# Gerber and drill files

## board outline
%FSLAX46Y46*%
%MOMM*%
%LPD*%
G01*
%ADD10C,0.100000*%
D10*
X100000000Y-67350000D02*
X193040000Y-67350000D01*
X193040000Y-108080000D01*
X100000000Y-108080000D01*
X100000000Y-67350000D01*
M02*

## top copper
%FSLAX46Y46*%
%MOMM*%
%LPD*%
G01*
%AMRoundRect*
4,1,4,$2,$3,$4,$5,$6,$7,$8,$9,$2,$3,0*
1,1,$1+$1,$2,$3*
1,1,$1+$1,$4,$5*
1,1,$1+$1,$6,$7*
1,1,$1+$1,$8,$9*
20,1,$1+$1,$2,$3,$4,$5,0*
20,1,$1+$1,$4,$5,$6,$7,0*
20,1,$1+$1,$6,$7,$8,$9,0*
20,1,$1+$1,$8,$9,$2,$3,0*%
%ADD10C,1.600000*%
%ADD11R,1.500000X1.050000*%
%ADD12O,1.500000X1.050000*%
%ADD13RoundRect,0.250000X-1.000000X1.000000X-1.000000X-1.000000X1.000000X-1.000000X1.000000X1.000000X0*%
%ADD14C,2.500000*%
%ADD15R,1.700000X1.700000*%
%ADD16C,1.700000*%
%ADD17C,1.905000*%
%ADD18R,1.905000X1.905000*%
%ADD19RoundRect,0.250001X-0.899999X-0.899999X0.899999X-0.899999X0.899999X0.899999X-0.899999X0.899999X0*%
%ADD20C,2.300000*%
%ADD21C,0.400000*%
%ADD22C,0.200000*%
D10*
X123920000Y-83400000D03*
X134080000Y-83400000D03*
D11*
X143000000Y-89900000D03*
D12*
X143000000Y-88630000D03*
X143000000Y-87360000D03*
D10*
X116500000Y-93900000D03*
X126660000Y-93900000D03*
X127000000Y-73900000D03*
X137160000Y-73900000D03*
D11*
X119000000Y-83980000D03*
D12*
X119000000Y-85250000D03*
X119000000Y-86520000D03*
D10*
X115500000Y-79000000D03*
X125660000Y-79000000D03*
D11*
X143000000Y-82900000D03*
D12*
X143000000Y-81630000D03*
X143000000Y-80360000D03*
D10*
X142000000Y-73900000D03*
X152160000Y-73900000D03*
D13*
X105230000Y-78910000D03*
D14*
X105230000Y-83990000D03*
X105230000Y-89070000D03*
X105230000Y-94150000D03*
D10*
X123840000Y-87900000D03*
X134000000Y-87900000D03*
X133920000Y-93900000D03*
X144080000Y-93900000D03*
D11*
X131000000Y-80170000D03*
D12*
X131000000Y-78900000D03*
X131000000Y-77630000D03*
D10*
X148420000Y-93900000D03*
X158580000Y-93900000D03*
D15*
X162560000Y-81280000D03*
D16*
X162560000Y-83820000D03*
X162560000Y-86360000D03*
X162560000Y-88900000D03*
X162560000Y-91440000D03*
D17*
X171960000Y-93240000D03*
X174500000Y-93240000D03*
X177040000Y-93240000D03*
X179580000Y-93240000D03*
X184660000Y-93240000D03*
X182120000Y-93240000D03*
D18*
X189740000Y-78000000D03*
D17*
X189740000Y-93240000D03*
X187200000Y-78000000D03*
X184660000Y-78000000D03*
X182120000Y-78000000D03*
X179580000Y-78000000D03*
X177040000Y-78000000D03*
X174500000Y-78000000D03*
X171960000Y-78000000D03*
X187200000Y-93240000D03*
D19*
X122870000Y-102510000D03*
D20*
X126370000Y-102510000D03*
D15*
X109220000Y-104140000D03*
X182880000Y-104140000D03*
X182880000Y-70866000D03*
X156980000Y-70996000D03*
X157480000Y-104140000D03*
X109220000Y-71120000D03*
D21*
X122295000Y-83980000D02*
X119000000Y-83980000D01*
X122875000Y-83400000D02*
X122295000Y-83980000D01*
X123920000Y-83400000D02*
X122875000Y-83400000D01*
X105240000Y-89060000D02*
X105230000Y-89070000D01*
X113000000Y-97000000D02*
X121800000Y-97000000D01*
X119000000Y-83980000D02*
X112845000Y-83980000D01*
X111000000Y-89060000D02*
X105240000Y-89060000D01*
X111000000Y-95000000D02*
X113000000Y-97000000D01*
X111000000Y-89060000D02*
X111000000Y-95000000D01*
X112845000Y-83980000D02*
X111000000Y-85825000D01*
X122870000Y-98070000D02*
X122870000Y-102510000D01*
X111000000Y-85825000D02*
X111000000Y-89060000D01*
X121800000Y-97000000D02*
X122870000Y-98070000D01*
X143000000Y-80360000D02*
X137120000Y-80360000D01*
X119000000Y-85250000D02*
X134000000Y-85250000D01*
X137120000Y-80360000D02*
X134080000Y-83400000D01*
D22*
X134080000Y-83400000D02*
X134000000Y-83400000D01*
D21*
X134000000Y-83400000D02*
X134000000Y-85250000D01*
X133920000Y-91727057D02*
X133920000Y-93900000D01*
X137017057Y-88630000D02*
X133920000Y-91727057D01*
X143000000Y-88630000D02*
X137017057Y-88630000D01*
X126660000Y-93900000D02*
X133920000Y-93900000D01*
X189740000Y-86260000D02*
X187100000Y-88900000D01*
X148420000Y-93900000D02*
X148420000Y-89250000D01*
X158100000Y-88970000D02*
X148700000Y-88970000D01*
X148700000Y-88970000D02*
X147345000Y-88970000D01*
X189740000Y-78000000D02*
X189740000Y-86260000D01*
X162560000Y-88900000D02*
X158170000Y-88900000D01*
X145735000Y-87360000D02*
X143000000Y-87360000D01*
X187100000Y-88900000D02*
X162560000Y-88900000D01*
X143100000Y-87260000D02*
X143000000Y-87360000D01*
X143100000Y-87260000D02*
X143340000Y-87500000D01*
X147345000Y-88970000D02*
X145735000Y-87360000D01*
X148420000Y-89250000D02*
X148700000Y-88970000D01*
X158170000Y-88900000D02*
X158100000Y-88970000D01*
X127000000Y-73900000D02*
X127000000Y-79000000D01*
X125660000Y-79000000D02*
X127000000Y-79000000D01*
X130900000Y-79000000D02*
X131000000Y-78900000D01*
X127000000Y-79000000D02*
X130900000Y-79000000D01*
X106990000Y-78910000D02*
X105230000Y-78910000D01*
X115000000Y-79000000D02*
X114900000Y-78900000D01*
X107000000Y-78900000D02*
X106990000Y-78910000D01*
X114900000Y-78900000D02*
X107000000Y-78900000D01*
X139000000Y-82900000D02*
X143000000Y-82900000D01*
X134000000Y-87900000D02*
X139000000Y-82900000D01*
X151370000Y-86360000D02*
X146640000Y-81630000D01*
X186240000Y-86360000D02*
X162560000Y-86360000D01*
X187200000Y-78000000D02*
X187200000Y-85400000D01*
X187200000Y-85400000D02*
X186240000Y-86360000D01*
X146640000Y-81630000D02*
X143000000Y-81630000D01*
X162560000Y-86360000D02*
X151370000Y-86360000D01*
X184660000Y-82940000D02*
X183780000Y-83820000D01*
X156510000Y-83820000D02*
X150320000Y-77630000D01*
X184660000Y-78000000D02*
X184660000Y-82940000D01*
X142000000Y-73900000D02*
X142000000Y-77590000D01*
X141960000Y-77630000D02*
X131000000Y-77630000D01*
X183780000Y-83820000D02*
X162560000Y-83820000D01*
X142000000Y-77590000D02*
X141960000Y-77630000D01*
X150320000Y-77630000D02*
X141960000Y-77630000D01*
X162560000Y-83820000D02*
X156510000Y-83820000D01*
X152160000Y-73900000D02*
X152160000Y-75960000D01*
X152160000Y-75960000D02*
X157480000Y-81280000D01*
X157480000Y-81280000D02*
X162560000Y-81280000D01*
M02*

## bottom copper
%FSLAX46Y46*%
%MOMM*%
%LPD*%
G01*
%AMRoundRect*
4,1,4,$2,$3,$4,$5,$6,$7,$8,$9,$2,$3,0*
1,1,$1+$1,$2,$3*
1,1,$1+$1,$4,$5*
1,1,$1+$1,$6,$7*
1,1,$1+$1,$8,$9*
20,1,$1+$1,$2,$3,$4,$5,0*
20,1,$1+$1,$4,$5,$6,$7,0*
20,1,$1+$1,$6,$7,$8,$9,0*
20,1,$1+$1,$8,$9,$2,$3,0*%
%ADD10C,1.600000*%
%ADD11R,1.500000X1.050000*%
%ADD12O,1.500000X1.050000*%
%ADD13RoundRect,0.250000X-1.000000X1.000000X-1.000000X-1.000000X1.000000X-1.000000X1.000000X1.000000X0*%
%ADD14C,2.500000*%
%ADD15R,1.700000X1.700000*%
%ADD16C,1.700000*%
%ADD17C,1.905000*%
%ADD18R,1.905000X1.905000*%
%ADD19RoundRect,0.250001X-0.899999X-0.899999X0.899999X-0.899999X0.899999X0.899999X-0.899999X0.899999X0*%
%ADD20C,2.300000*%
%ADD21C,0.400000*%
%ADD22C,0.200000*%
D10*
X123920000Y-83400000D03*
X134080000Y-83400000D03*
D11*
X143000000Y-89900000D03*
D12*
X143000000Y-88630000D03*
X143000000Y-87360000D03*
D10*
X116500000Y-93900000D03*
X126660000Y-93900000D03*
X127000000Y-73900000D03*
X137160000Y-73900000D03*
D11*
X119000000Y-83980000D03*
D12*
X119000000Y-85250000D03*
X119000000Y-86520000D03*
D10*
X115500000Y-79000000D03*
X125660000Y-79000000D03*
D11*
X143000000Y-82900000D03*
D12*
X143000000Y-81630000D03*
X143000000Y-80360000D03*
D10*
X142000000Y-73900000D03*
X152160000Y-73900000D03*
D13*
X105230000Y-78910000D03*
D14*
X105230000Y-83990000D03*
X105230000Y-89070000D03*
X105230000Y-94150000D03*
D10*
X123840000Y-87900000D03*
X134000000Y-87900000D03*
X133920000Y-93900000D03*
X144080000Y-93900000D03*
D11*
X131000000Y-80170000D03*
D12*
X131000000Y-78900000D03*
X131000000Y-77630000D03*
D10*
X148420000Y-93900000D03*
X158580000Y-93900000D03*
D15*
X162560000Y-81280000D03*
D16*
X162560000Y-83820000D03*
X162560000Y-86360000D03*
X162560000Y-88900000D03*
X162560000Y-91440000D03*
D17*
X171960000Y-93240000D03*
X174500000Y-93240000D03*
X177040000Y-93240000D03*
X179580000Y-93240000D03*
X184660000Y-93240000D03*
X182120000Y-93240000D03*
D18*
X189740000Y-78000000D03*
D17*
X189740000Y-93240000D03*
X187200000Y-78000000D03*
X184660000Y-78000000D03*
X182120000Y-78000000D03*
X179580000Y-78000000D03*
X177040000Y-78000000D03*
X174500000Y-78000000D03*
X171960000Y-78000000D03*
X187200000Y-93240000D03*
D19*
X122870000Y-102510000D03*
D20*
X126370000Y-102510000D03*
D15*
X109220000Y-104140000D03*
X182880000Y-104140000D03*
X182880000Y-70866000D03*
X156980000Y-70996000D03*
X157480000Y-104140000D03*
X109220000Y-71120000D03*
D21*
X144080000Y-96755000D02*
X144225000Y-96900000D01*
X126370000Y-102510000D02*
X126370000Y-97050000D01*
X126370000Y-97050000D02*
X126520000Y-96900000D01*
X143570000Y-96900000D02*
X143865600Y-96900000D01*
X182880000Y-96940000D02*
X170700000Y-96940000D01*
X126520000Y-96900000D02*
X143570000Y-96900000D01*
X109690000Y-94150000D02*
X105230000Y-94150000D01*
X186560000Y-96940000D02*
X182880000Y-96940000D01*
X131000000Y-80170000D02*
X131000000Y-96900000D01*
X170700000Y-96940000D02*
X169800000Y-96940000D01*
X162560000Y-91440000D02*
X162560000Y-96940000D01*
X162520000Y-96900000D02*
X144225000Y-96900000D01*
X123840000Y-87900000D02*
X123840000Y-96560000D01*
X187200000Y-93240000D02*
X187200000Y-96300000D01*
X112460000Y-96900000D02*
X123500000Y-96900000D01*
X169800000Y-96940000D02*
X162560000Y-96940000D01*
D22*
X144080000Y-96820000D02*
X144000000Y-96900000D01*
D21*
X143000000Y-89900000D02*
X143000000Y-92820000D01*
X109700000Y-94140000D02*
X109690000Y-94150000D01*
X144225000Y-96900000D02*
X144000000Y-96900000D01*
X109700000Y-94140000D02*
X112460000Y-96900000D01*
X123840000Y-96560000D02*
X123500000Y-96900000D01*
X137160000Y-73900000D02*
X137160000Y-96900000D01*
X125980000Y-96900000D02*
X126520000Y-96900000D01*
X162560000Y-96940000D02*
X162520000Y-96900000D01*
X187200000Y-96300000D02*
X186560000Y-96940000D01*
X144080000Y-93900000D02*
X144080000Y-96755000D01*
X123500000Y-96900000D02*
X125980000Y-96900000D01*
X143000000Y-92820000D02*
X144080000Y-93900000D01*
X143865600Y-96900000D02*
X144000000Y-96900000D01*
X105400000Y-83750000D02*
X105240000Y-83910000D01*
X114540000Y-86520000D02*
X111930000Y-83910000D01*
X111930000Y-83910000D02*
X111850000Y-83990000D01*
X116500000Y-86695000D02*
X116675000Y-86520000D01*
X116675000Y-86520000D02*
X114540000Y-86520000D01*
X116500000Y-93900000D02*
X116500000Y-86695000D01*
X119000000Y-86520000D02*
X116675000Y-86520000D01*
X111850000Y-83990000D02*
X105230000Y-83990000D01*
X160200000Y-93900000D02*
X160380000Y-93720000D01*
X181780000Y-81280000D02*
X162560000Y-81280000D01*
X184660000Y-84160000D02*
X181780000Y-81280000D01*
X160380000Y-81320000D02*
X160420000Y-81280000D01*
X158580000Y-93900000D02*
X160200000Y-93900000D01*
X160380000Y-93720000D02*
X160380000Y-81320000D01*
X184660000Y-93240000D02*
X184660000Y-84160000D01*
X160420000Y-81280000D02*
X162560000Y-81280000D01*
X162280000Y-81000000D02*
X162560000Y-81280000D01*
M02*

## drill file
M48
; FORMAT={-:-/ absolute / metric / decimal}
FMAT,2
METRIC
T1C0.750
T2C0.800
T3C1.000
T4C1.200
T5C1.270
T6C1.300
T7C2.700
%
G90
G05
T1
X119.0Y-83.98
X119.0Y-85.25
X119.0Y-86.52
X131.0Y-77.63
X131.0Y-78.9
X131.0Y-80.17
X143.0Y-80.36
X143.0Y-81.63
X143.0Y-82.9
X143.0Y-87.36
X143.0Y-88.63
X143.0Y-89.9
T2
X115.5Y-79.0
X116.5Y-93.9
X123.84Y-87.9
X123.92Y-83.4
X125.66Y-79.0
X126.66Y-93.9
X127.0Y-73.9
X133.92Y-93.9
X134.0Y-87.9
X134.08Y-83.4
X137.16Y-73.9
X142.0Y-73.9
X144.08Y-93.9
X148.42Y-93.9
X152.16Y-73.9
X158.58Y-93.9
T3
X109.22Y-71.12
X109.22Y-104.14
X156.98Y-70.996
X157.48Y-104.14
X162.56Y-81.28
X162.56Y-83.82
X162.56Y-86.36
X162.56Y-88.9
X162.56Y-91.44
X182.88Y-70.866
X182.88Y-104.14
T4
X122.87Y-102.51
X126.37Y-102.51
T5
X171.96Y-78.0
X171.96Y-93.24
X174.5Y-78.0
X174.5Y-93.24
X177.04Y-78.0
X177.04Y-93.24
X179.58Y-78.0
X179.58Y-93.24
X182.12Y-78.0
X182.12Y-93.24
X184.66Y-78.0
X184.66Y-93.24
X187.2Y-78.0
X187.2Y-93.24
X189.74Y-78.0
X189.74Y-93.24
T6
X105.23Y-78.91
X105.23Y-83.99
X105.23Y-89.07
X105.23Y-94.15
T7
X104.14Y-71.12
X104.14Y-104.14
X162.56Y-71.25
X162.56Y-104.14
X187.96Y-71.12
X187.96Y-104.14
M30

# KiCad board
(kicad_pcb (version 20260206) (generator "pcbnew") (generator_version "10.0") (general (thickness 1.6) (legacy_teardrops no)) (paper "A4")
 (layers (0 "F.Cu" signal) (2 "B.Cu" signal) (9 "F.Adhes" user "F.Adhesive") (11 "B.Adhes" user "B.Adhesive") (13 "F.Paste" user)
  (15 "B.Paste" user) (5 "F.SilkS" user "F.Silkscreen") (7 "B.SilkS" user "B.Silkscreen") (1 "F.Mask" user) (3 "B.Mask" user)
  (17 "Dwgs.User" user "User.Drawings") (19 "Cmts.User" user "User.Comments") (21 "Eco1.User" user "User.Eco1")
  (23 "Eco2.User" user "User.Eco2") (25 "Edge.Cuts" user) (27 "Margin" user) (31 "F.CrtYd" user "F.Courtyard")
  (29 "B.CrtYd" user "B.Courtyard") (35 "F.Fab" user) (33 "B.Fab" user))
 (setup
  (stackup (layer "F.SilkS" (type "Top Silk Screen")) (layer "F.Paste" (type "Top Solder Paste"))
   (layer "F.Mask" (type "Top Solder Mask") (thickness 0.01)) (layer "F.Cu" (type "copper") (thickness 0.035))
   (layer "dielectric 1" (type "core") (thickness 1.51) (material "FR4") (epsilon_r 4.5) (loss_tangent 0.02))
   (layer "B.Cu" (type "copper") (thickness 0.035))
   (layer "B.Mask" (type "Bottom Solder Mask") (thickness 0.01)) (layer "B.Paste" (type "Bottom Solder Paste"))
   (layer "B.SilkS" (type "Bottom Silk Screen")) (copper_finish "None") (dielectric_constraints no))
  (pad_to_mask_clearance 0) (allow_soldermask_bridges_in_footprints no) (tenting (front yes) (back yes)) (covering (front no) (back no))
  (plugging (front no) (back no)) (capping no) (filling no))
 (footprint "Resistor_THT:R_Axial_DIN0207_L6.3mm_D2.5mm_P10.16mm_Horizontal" (layer "F.Cu") (at 123.92 83.4)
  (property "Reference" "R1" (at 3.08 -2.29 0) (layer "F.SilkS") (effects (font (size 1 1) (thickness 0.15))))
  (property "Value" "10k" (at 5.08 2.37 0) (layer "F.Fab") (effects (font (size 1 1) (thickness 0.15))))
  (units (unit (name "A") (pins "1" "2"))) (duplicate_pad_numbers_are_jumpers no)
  (pad "1" thru_hole circle (at 0 0) (size 1.6 1.6) (drill 0.8) (layers "*.Cu" "*.Mask") (remove_unused_layers no) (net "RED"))
  (pad "2" thru_hole circle (at 10.16 0) (size 1.6 1.6) (drill 0.8) (layers "*.Cu" "*.Mask") (remove_unused_layers no) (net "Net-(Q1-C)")))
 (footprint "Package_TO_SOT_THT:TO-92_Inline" (layer "F.Cu") (at 143 89.9 90)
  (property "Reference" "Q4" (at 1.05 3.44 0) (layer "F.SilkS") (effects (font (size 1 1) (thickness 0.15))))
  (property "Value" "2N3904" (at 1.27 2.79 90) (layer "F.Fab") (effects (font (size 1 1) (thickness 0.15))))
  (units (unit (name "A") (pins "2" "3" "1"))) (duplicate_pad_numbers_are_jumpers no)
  (pad "1" thru_hole rect (at 0 0 90) (size 1.05 1.5) (drill 0.75) (layers "*.Cu" "*.Mask") (remove_unused_layers no) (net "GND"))
  (pad "2" thru_hole oval (at 1.27 0 90) (size 1.05 1.5) (drill 0.75) (layers "*.Cu" "*.Mask") (remove_unused_layers no) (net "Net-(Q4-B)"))
  (pad "3" thru_hole oval (at 2.54 0 90) (size 1.05 1.5) (drill 0.75) (layers "*.Cu" "*.Mask") (remove_unused_layers no) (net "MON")))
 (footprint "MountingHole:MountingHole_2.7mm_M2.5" (layer "F.Cu") (at 187.96 104.14)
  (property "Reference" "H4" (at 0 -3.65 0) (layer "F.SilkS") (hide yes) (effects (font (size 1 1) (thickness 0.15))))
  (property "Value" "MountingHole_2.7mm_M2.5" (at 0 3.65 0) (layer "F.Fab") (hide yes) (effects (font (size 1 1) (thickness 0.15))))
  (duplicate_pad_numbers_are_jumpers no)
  (pad "" np_thru_hole circle (at 0 0) (size 2.7 2.7) (drill 2.7) (layers "*.Cu" "*.Mask")))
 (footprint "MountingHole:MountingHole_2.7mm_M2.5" (layer "F.Cu") (at 162.56 104.14)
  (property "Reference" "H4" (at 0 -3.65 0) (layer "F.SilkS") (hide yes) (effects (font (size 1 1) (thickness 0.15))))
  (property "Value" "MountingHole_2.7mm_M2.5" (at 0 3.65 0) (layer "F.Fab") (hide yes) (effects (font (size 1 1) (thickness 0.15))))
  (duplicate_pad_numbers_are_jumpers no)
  (pad "" np_thru_hole circle (at 0 0) (size 2.7 2.7) (drill 2.7) (layers "*.Cu" "*.Mask")))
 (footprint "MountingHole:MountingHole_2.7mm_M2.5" (layer "F.Cu") (at 104.14 71.12)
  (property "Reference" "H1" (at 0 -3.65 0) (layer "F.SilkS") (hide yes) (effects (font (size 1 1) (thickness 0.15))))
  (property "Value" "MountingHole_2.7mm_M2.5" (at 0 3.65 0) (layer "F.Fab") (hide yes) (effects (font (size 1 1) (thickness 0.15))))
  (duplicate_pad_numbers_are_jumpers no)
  (pad "" np_thru_hole circle (at 0 0) (size 2.7 2.7) (drill 2.7) (layers "*.Cu" "*.Mask")))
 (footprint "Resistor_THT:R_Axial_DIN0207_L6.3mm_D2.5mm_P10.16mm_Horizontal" (layer "F.Cu") (at 116.5 93.9)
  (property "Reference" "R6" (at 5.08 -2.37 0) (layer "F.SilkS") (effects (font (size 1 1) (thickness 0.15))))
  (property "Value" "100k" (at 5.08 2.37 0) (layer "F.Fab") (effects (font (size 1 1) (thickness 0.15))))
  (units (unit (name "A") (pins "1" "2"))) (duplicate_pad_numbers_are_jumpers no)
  (pad "1" thru_hole circle (at 0 0) (size 1.6 1.6) (drill 0.8) (layers "*.Cu" "*.Mask") (remove_unused_layers no) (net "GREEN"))
  (pad "2" thru_hole circle (at 10.16 0) (size 1.6 1.6) (drill 0.8) (layers "*.Cu" "*.Mask") (remove_unused_layers no) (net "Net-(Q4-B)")))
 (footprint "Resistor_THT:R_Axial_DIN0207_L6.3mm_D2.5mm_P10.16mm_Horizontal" (layer "F.Cu") (at 127 73.9)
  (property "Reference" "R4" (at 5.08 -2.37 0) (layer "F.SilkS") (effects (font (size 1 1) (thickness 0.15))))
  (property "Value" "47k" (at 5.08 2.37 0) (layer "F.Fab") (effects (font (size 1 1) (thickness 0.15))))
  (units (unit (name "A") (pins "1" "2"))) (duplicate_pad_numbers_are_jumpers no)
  (pad "1" thru_hole circle (at 0 0) (size 1.6 1.6) (drill 0.8) (layers "*.Cu" "*.Mask") (remove_unused_layers no) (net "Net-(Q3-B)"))
  (pad "2" thru_hole circle (at 10.16 0) (size 1.6 1.6) (drill 0.8) (layers "*.Cu" "*.Mask") (remove_unused_layers no) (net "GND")))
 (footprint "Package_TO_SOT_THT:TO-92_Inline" (layer "F.Cu") (at 119 83.98 -90)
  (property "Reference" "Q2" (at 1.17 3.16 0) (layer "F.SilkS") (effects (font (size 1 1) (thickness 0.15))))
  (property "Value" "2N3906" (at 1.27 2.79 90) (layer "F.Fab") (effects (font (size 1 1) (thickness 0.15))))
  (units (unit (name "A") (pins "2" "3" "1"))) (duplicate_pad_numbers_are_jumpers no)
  (pad "1" thru_hole rect (at 0 0 270) (size 1.05 1.5) (drill 0.75) (layers "*.Cu" "*.Mask") (remove_unused_layers no) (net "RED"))
  (pad "2" thru_hole oval (at 1.27 0 270) (size 1.05 1.5) (drill 0.75) (layers "*.Cu" "*.Mask") (remove_unused_layers no) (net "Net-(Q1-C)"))
  (pad "3" thru_hole oval (at 2.54 0 270) (size 1.05 1.5) (drill 0.75) (layers "*.Cu" "*.Mask") (remove_unused_layers no) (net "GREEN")))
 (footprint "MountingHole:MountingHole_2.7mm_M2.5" (layer "F.Cu") (at 162.56 71.25)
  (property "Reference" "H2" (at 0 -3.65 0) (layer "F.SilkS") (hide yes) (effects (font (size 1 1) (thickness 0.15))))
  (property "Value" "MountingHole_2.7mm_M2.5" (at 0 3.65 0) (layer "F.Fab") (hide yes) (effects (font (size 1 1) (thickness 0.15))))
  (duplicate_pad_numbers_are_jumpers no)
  (pad "" np_thru_hole circle (at 0 0) (size 2.7 2.7) (drill 2.7) (layers "*.Cu" "*.Mask")))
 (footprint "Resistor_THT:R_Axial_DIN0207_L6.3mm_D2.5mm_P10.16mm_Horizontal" (layer "F.Cu") (at 115.5 79)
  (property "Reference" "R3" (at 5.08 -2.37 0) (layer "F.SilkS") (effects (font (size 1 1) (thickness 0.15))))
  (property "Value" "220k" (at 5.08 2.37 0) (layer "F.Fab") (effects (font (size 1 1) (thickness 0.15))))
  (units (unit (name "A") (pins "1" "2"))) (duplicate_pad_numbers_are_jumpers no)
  (pad "1" thru_hole circle (at 0 0) (size 1.6 1.6) (drill 0.8) (layers "*.Cu" "*.Mask") (remove_unused_layers no) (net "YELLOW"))
  (pad "2" thru_hole circle (at 10.16 0) (size 1.6 1.6) (drill 0.8) (layers "*.Cu" "*.Mask") (remove_unused_layers no) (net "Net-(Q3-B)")))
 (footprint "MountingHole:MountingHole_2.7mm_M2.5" (layer "F.Cu") (at 187.96 71.12)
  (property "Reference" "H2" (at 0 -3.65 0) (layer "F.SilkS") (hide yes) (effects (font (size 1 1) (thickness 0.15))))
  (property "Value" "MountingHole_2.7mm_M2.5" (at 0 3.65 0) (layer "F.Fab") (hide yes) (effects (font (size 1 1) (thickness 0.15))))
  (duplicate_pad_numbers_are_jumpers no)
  (pad "" np_thru_hole circle (at 0 0) (size 2.7 2.7) (drill 2.7) (layers "*.Cu" "*.Mask")))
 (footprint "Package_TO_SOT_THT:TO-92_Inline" (layer "F.Cu") (at 143 82.9 90)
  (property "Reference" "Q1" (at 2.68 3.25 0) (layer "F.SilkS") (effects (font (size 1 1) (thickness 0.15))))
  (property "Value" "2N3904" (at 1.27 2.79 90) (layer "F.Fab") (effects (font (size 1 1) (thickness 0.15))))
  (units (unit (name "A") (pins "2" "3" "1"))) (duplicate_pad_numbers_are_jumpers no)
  (pad "1" thru_hole rect (at 0 0 90) (size 1.05 1.5) (drill 0.75) (layers "*.Cu" "*.Mask") (remove_unused_layers no) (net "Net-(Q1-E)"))
  (pad "2" thru_hole oval (at 1.27 0 90) (size 1.05 1.5) (drill 0.75) (layers "*.Cu" "*.Mask") (remove_unused_layers no) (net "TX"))
  (pad "3" thru_hole oval (at 2.54 0 90) (size 1.05 1.5) (drill 0.75) (layers "*.Cu" "*.Mask") (remove_unused_layers no) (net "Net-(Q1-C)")))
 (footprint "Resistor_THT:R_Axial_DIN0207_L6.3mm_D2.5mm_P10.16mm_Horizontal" (layer "F.Cu") (at 142 73.9)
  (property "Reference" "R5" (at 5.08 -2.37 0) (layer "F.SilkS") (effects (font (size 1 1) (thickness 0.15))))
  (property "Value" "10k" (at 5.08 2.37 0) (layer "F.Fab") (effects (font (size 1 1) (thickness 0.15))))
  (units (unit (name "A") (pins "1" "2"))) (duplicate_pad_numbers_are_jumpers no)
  (pad "1" thru_hole circle (at 0 0) (size 1.6 1.6) (drill 0.8) (layers "*.Cu" "*.Mask") (remove_unused_layers no) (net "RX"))
  (pad "2" thru_hole circle (at 10.16 0) (size 1.6 1.6) (drill 0.8) (layers "*.Cu" "*.Mask") (remove_unused_layers no) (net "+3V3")))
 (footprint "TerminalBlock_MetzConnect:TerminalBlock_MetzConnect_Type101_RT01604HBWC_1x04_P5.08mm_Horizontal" (layer "F.Cu")
  (at 105.23 78.91 -90)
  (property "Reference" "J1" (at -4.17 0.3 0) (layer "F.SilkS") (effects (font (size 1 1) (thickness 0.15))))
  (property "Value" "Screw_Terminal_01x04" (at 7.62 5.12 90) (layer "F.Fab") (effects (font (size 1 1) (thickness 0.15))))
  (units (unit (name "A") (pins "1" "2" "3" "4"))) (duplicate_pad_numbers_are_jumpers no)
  (pad "1" thru_hole roundrect (at 0 0 270) (size 2.5 2.5) (drill 1.3) (layers "*.Cu" "*.Mask") (remove_unused_layers no)
   (roundrect_rratio 0.1) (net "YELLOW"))
  (pad "2" thru_hole circle (at 5.08 0 270) (size 2.5 2.5) (drill 1.3) (layers "*.Cu" "*.Mask") (remove_unused_layers no) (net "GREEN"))
  (pad "3" thru_hole circle (at 10.16 0 270) (size 2.5 2.5) (drill 1.3) (layers "*.Cu" "*.Mask") (remove_unused_layers no) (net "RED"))
  (pad "4" thru_hole circle (at 15.24 0 270) (size 2.5 2.5) (drill 1.3) (layers "*.Cu" "*.Mask") (remove_unused_layers no) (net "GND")))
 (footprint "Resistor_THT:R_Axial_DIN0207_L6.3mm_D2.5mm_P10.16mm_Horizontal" (layer "F.Cu") (at 123.84 87.9)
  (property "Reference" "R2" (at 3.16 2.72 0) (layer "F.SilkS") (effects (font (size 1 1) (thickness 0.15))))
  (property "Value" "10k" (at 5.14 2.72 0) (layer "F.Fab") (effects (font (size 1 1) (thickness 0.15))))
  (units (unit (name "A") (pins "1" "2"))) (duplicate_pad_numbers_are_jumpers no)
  (pad "1" thru_hole circle (at 0 0) (size 1.6 1.6) (drill 0.8) (layers "*.Cu" "*.Mask") (remove_unused_layers no) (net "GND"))
  (pad "2" thru_hole circle (at 10.16 0) (size 1.6 1.6) (drill 0.8) (layers "*.Cu" "*.Mask") (remove_unused_layers no) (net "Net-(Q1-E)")))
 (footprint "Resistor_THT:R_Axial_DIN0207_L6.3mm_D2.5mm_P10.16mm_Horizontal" (layer "F.Cu") (at 133.92 93.9)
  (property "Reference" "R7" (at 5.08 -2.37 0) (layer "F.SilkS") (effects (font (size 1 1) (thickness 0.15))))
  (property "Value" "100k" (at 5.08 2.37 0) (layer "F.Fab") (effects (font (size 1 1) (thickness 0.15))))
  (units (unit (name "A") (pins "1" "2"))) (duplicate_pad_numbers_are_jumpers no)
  (pad "1" thru_hole circle (at 0 0) (size 1.6 1.6) (drill 0.8) (layers "*.Cu" "*.Mask") (remove_unused_layers no) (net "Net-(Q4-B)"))
  (pad "2" thru_hole circle (at 10.16 0) (size 1.6 1.6) (drill 0.8) (layers "*.Cu" "*.Mask") (remove_unused_layers no) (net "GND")))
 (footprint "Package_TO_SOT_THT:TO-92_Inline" (layer "F.Cu") (at 131 80.17 90)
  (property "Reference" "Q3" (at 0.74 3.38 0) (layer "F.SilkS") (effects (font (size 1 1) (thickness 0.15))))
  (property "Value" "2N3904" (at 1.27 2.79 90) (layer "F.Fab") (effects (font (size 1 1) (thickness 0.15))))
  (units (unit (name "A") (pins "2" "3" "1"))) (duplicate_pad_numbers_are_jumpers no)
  (pad "1" thru_hole rect (at 0 0 90) (size 1.05 1.5) (drill 0.75) (layers "*.Cu" "*.Mask") (remove_unused_layers no) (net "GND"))
  (pad "2" thru_hole oval (at 1.27 0 90) (size 1.05 1.5) (drill 0.75) (layers "*.Cu" "*.Mask") (remove_unused_layers no) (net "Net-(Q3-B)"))
  (pad "3" thru_hole oval (at 2.54 0 90) (size 1.05 1.5) (drill 0.75) (layers "*.Cu" "*.Mask") (remove_unused_layers no) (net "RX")))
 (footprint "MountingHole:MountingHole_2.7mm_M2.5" (layer "F.Cu") (at 104.14 104.14)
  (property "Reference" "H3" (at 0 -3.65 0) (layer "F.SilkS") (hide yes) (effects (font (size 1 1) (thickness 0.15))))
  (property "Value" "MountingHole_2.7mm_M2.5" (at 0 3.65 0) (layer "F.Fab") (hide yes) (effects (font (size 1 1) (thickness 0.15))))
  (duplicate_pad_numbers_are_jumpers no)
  (pad "" np_thru_hole circle (at 0 0) (size 2.7 2.7) (drill 2.7) (layers "*.Cu" "*.Mask")))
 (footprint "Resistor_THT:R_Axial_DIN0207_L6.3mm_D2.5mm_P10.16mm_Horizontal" (layer "F.Cu") (at 148.42 93.9)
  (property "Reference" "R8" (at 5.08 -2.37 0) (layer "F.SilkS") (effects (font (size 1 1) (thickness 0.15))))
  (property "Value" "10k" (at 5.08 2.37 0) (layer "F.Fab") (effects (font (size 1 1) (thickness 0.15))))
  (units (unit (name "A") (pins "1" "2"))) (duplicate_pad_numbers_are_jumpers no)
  (pad "1" thru_hole circle (at 0 0) (size 1.6 1.6) (drill 0.8) (layers "*.Cu" "*.Mask") (remove_unused_layers no) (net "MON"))
  (pad "2" thru_hole circle (at 10.16 0) (size 1.6 1.6) (drill 0.8) (layers "*.Cu" "*.Mask") (remove_unused_layers no) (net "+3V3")))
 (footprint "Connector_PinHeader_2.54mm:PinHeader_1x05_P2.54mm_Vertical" (layer "F.Cu") (at 162.56 81.28)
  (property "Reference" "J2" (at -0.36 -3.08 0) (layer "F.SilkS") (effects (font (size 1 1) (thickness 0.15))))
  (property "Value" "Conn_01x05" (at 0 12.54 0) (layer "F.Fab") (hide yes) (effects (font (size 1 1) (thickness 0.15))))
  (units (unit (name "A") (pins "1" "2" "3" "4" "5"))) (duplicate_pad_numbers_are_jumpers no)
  (pad "1" thru_hole rect (at 0 0) (size 1.7 1.7) (drill 1) (layers "*.Cu" "*.Mask") (remove_unused_layers no) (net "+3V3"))
  (pad "2" thru_hole circle (at 0 2.54) (size 1.7 1.7) (drill 1) (layers "*.Cu" "*.Mask") (remove_unused_layers no) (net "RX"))
  (pad "3" thru_hole circle (at 0 5.08) (size 1.7 1.7) (drill 1) (layers "*.Cu" "*.Mask") (remove_unused_layers no) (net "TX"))
  (pad "4" thru_hole circle (at 0 7.62) (size 1.7 1.7) (drill 1) (layers "*.Cu" "*.Mask") (remove_unused_layers no) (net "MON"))
  (pad "5" thru_hole circle (at 0 10.16) (size 1.7 1.7) (drill 1) (layers "*.Cu" "*.Mask") (remove_unused_layers no) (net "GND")))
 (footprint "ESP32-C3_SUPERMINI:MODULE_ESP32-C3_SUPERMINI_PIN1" (layer "F.Cu") (at 179.84 85.62 -90)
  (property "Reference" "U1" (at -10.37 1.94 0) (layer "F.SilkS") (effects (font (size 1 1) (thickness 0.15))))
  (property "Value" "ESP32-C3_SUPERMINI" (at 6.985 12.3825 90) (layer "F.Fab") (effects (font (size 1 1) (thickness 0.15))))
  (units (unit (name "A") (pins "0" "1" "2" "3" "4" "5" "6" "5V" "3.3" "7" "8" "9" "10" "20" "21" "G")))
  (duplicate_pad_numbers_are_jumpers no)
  (pad "0" thru_hole circle (at 7.62 7.88 270) (size 1.905 1.905) (drill 1.27) (layers "*.Cu" "*.Mask") (remove_unused_layers no)
   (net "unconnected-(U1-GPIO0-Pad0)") (solder_mask_margin 0.102))
  (pad "1" thru_hole circle (at 7.62 5.34 270) (size 1.905 1.905) (drill 1.27) (layers "*.Cu" "*.Mask") (remove_unused_layers no)
   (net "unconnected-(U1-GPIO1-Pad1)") (solder_mask_margin 0.102))
  (pad "2" thru_hole circle (at 7.62 2.8 270) (size 1.905 1.905) (drill 1.27) (layers "*.Cu" "*.Mask") (remove_unused_layers no)
   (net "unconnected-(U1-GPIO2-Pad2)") (solder_mask_margin 0.102))
  (pad "3" thru_hole circle (at 7.62 0.26 270) (size 1.905 1.905) (drill 1.27) (layers "*.Cu" "*.Mask") (remove_unused_layers no)
   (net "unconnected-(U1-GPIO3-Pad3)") (solder_mask_margin 0.102))
  (pad "3.3" thru_hole circle (at 7.62 -4.82 270) (size 1.905 1.905) (drill 1.27) (layers "*.Cu" "*.Mask") (remove_unused_layers no)
   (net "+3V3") (solder_mask_margin 0.102))
  (pad "4" thru_hole circle (at 7.62 -2.28 270) (size 1.905 1.905) (drill 1.27) (layers "*.Cu" "*.Mask") (remove_unused_layers no)
   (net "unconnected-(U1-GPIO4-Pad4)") (solder_mask_margin 0.102))
  (pad "5" thru_hole rect (at -7.62 -9.9 270) (size 1.905 1.905) (drill 1.27) (layers "*.Cu" "*.Mask") (remove_unused_layers no) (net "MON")
   (solder_mask_margin 0.102))
  (pad "5V" thru_hole circle (at 7.62 -9.9 270) (size 1.905 1.905) (drill 1.27) (layers "*.Cu" "*.Mask") (remove_unused_layers no)
   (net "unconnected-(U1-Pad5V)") (solder_mask_margin 0.102))
  (pad "6" thru_hole circle (at -7.62 -7.36 270) (size 1.905 1.905) (drill 1.27) (layers "*.Cu" "*.Mask") (remove_unused_layers no)
   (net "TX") (solder_mask_margin 0.102))
  (pad "7" thru_hole circle (at -7.62 -4.82 270) (size 1.905 1.905) (drill 1.27) (layers "*.Cu" "*.Mask") (remove_unused_layers no)
   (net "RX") (solder_mask_margin 0.102))
  (pad "8" thru_hole circle (at -7.62 -2.28 270) (size 1.905 1.905) (drill 1.27) (layers "*.Cu" "*.Mask") (remove_unused_layers no)
   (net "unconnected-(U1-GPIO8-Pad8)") (solder_mask_margin 0.102))
  (pad "9" thru_hole circle (at -7.62 0.26 270) (size 1.905 1.905) (drill 1.27) (layers "*.Cu" "*.Mask") (remove_unused_layers no)
   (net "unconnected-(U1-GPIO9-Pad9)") (solder_mask_margin 0.102))
  (pad "10" thru_hole circle (at -7.62 2.8 270) (size 1.905 1.905) (drill 1.27) (layers "*.Cu" "*.Mask") (remove_unused_layers no)
   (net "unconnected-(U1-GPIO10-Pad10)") (solder_mask_margin 0.102))
  (pad "20" thru_hole circle (at -7.62 5.34 270) (size 1.905 1.905) (drill 1.27) (layers "*.Cu" "*.Mask") (remove_unused_layers no)
   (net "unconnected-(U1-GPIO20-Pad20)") (solder_mask_margin 0.102))
  (pad "21" thru_hole circle (at -7.62 7.88 270) (size 1.905 1.905) (drill 1.27) (layers "*.Cu" "*.Mask") (remove_unused_layers no)
   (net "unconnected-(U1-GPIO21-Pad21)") (solder_mask_margin 0.102))
  (pad "G" thru_hole circle (at 7.62 -7.36 270) (size 1.905 1.905) (drill 1.27) (layers "*.Cu" "*.Mask") (remove_unused_layers no)
   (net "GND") (solder_mask_margin 0.102)))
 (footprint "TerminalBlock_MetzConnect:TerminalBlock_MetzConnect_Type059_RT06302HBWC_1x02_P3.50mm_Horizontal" (layer "F.Cu")
  (at 122.87 102.51)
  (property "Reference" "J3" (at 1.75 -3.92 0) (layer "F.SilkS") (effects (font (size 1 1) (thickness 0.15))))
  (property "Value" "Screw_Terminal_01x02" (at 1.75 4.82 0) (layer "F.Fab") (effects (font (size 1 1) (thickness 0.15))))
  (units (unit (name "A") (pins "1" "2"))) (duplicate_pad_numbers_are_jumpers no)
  (pad "1" thru_hole roundrect (at 0 0) (size 2.3 2.3) (drill 1.2) (layers "*.Cu" "*.Mask") (remove_unused_layers no)
   (roundrect_rratio 0.108696) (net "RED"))
  (pad "2" thru_hole circle (at 3.5 0) (size 2.3 2.3) (drill 1.2) (layers "*.Cu" "*.Mask") (remove_unused_layers no) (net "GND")))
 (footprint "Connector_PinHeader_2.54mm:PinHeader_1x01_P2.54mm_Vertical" (layer "B.Cu") (at 109.22 104.14)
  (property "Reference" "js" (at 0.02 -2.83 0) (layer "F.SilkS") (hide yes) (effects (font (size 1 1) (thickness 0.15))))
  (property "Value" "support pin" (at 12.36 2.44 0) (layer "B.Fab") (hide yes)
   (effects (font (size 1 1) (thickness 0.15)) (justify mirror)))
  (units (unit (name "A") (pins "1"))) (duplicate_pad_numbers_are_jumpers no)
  (pad "1" thru_hole rect (at 0 0) (size 1.7 1.7) (drill 1) (layers "*.Cu" "*.Mask") (remove_unused_layers no)
   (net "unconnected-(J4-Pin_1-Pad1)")))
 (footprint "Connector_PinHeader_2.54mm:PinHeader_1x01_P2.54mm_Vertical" (layer "B.Cu") (at 182.88 104.14)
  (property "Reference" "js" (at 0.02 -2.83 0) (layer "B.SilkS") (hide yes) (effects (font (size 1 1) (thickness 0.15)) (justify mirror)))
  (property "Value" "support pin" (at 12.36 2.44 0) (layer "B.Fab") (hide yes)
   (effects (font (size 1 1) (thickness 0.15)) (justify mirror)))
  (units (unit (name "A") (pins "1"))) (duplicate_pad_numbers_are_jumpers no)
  (pad "1" thru_hole rect (at 0 0) (size 1.7 1.7) (drill 1) (layers "*.Cu" "*.Mask") (remove_unused_layers no)
   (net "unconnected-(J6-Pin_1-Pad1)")))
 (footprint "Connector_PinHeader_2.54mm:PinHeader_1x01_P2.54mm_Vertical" (layer "B.Cu") (at 182.88 70.866)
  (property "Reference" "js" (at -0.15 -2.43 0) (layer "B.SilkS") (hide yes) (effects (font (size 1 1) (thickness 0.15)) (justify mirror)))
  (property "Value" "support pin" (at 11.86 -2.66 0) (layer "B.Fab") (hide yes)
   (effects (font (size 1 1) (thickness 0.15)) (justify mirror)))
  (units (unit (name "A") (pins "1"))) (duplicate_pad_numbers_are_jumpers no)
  (pad "1" thru_hole rect (at 0 0) (size 1.7 1.7) (drill 1) (layers "*.Cu" "*.Mask") (remove_unused_layers no)
   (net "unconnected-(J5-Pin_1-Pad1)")))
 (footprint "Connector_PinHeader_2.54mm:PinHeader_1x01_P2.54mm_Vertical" (layer "B.Cu") (at 156.98 70.996)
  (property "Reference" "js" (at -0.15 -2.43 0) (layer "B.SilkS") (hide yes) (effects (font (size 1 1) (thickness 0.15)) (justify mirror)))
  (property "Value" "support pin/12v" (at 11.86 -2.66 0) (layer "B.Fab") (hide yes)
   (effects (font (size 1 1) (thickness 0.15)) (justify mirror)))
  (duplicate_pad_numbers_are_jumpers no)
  (pad "1" thru_hole rect (at 0 0) (size 1.7 1.7) (drill 1) (layers "*.Cu" "*.Mask") (remove_unused_layers no)))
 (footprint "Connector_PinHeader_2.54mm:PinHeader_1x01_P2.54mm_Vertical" (layer "B.Cu") (at 157.48 104.14)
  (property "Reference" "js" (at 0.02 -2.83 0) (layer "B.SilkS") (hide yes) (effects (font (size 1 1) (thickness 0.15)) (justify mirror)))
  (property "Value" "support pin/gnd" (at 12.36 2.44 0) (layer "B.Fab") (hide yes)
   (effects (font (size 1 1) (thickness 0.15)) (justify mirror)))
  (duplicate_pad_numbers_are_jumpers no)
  (pad "1" thru_hole rect (at 0 0) (size 1.7 1.7) (drill 1) (layers "*.Cu" "*.Mask") (remove_unused_layers no)))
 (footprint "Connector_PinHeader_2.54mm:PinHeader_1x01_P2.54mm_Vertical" (layer "B.Cu") (at 109.22 71.12)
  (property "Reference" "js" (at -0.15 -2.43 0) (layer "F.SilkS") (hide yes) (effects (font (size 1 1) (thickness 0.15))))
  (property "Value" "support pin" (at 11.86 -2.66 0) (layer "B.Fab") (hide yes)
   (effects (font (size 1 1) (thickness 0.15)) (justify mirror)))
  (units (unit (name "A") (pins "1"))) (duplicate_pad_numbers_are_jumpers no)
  (pad "1" thru_hole rect (at 0 0) (size 1.7 1.7) (drill 1) (layers "*.Cu" "*.Mask") (remove_unused_layers no)
   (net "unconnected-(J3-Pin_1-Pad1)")))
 (gr_rect (start 100 67.35) (end 193.04 108.08) (stroke (width 0.1) (type default)) (fill no) (layer "Edge.Cuts"))
 (segment (start 122.295 83.98) (end 119 83.98) (width 0.4) (layer "F.Cu") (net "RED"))
 (segment (start 122.875 83.4) (end 122.295 83.98) (width 0.4) (layer "F.Cu") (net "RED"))
 (segment (start 123.92 83.4) (end 122.875 83.4) (width 0.4) (layer "F.Cu") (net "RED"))
 (segment (start 105.24 89.06) (end 105.23 89.07) (width 0.4) (layer "F.Cu") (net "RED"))
 (segment (start 113 97) (end 121.8 97) (width 0.4) (layer "F.Cu") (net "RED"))
 (segment (start 119 83.98) (end 112.845 83.98) (width 0.4) (layer "F.Cu") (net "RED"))
 (segment (start 111 89.06) (end 105.24 89.06) (width 0.4) (layer "F.Cu") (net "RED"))
 (segment (start 111 95) (end 113 97) (width 0.4) (layer "F.Cu") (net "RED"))
 (segment (start 111 89.06) (end 111 95) (width 0.4) (layer "F.Cu") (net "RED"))
 (segment (start 112.845 83.98) (end 111 85.825) (width 0.4) (layer "F.Cu") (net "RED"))
 (segment (start 122.87 98.07) (end 122.87 102.51) (width 0.4) (layer "F.Cu") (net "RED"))
 (segment (start 111 85.825) (end 111 89.06) (width 0.4) (layer "F.Cu") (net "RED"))
 (segment (start 121.8 97) (end 122.87 98.07) (width 0.4) (layer "F.Cu") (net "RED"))
 (segment (start 143 80.36) (end 137.12 80.36) (width 0.4) (layer "F.Cu") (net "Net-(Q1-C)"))
 (segment (start 119 85.25) (end 134 85.25) (width 0.4) (layer "F.Cu") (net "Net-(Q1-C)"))
 (segment (start 137.12 80.36) (end 134.08 83.4) (width 0.4) (layer "F.Cu") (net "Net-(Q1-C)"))
 (segment (start 134.08 83.4) (end 134 83.4) (width 0.2) (layer "F.Cu") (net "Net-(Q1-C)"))
 (segment (start 134 83.4) (end 134 85.25) (width 0.4) (layer "F.Cu") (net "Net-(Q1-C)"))
 (segment (start 144.08 96.755) (end 144.225 96.9) (width 0.4) (layer "B.Cu") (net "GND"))
 (segment (start 126.37 102.51) (end 126.37 97.05) (width 0.4) (layer "B.Cu") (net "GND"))
 (segment (start 126.37 97.05) (end 126.52 96.9) (width 0.4) (layer "B.Cu") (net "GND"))
 (segment (start 143.57 96.9) (end 143.8656 96.9) (width 0.4) (layer "B.Cu") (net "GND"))
 (segment (start 182.88 96.94) (end 170.7 96.94) (width 0.4) (layer "B.Cu") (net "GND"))
 (segment (start 126.52 96.9) (end 143.57 96.9) (width 0.4) (layer "B.Cu") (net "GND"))
 (segment (start 109.69 94.15) (end 105.23 94.15) (width 0.4) (layer "B.Cu") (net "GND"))
 (segment (start 186.56 96.94) (end 182.88 96.94) (width 0.4) (layer "B.Cu") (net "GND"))
 (segment (start 131 80.17) (end 131 96.9) (width 0.4) (layer "B.Cu") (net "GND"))
 (segment (start 170.7 96.94) (end 169.8 96.94) (width 0.4) (layer "B.Cu") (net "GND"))
 (segment (start 162.56 91.44) (end 162.56 96.94) (width 0.4) (layer "B.Cu") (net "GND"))
 (segment (start 162.52 96.9) (end 144.225 96.9) (width 0.4) (layer "B.Cu") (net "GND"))
 (segment (start 123.84 87.9) (end 123.84 96.56) (width 0.4) (layer "B.Cu") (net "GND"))
 (segment (start 187.2 93.24) (end 187.2 96.3) (width 0.4) (layer "B.Cu") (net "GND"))
 (segment (start 112.46 96.9) (end 123.5 96.9) (width 0.4) (layer "B.Cu") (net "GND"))
 (segment (start 169.8 96.94) (end 162.56 96.94) (width 0.4) (layer "B.Cu") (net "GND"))
 (segment (start 144.08 96.82) (end 144 96.9) (width 0.2) (layer "B.Cu") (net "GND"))
 (segment (start 143 89.9) (end 143 92.82) (width 0.4) (layer "B.Cu") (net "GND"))
 (segment (start 109.7 94.14) (end 109.69 94.15) (width 0.4) (layer "B.Cu") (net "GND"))
 (segment (start 144.225 96.9) (end 144 96.9) (width 0.4) (layer "B.Cu") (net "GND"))
 (segment (start 109.7 94.14) (end 112.46 96.9) (width 0.4) (layer "B.Cu") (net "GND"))
 (segment (start 123.84 96.56) (end 123.5 96.9) (width 0.4) (layer "B.Cu") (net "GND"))
 (segment (start 137.16 73.9) (end 137.16 96.9) (width 0.4) (layer "B.Cu") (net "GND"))
 (segment (start 125.98 96.9) (end 126.52 96.9) (width 0.4) (layer "B.Cu") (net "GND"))
 (segment (start 162.56 96.94) (end 162.52 96.9) (width 0.4) (layer "B.Cu") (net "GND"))
 (segment (start 187.2 96.3) (end 186.56 96.94) (width 0.4) (layer "B.Cu") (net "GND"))
 (segment (start 144.08 93.9) (end 144.08 96.755) (width 0.4) (layer "B.Cu") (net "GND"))
 (segment (start 123.5 96.9) (end 125.98 96.9) (width 0.4) (layer "B.Cu") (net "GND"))
 (segment (start 143 92.82) (end 144.08 93.9) (width 0.4) (layer "B.Cu") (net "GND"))
 (segment (start 143.8656 96.9) (end 144 96.9) (width 0.4) (layer "B.Cu") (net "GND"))
 (segment (start 133.92 91.727057) (end 133.92 93.9) (width 0.4) (layer "F.Cu") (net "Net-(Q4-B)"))
 (segment (start 137.017057 88.63) (end 133.92 91.727057) (width 0.4) (layer "F.Cu") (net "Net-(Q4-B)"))
 (segment (start 143 88.63) (end 137.017057 88.63) (width 0.4) (layer "F.Cu") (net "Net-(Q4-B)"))
 (segment (start 126.66 93.9) (end 133.92 93.9) (width 0.4) (layer "F.Cu") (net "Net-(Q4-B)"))
 (segment (start 189.74 86.26) (end 187.1 88.9) (width 0.4) (layer "F.Cu") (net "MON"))
 (segment (start 148.42 93.9) (end 148.42 89.25) (width 0.4) (layer "F.Cu") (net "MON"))
 (segment (start 158.1 88.97) (end 148.7 88.97) (width 0.4) (layer "F.Cu") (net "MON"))
 (segment (start 148.7 88.97) (end 147.345 88.97) (width 0.4) (layer "F.Cu") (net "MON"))
 (segment (start 189.74 78) (end 189.74 86.26) (width 0.4) (layer "F.Cu") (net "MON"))
 (segment (start 162.56 88.9) (end 158.17 88.9) (width 0.4) (layer "F.Cu") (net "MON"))
 (segment (start 145.735 87.36) (end 143 87.36) (width 0.4) (layer "F.Cu") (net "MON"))
 (segment (start 187.1 88.9) (end 162.56 88.9) (width 0.4) (layer "F.Cu") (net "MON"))
 (segment (start 143.1 87.26) (end 143 87.36) (width 0.4) (layer "F.Cu") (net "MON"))
 (segment (start 143.1 87.26) (end 143.34 87.5) (width 0.4) (layer "F.Cu") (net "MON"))
 (segment (start 147.345 88.97) (end 145.735 87.36) (width 0.4) (layer "F.Cu") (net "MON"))
 (segment (start 148.42 89.25) (end 148.7 88.97) (width 0.4) (layer "F.Cu") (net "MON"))
 (segment (start 158.17 88.9) (end 158.1 88.97) (width 0.4) (layer "F.Cu") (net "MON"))
 (segment (start 105.4 83.75) (end 105.24 83.91) (width 0.4) (layer "B.Cu") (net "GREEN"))
 (segment (start 114.54 86.52) (end 111.93 83.91) (width 0.4) (layer "B.Cu") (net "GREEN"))
 (segment (start 111.93 83.91) (end 111.85 83.99) (width 0.4) (layer "B.Cu") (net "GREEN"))
 (segment (start 116.5 86.695) (end 116.675 86.52) (width 0.4) (layer "B.Cu") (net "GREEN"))
 (segment (start 116.675 86.52) (end 114.54 86.52) (width 0.4) (layer "B.Cu") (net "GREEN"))
 (segment (start 116.5 93.9) (end 116.5 86.695) (width 0.4) (layer "B.Cu") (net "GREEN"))
 (segment (start 119 86.52) (end 116.675 86.52) (width 0.4) (layer "B.Cu") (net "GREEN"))
 (segment (start 111.85 83.99) (end 105.23 83.99) (width 0.4) (layer "B.Cu") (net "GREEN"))
 (segment (start 127 73.9) (end 127 79) (width 0.4) (layer "F.Cu") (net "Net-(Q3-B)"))
 (segment (start 125.66 79) (end 127 79) (width 0.4) (layer "F.Cu") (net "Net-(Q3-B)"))
 (segment (start 130.9 79) (end 131 78.9) (width 0.4) (layer "F.Cu") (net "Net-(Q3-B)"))
 (segment (start 127 79) (end 130.9 79) (width 0.4) (layer "F.Cu") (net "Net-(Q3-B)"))
 (segment (start 106.99 78.91) (end 105.23 78.91) (width 0.4) (layer "F.Cu") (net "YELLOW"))
 (segment (start 115 79) (end 114.9 78.9) (width 0.4) (layer "F.Cu") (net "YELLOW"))
 (segment (start 107 78.9) (end 106.99 78.91) (width 0.4) (layer "F.Cu") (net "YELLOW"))
 (segment (start 114.9 78.9) (end 107 78.9) (width 0.4) (layer "F.Cu") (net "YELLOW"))
 (segment (start 139 82.9) (end 143 82.9) (width 0.4) (layer "F.Cu") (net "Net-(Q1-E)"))
 (segment (start 134 87.9) (end 139 82.9) (width 0.4) (layer "F.Cu") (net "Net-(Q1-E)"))
 (segment (start 151.37 86.36) (end 146.64 81.63) (width 0.4) (layer "F.Cu") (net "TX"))
 (segment (start 186.24 86.36) (end 162.56 86.36) (width 0.4) (layer "F.Cu") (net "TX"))
 (segment (start 187.2 78) (end 187.2 85.4) (width 0.4) (layer "F.Cu") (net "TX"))
 (segment (start 187.2 85.4) (end 186.24 86.36) (width 0.4) (layer "F.Cu") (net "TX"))
 (segment (start 146.64 81.63) (end 143 81.63) (width 0.4) (layer "F.Cu") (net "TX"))
 (segment (start 162.56 86.36) (end 151.37 86.36) (width 0.4) (layer "F.Cu") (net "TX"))
 (segment (start 184.66 82.94) (end 183.78 83.82) (width 0.4) (layer "F.Cu") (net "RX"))
 (segment (start 156.51 83.82) (end 150.32 77.63) (width 0.4) (layer "F.Cu") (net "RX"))
 (segment (start 184.66 78) (end 184.66 82.94) (width 0.4) (layer "F.Cu") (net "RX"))
 (segment (start 142 73.9) (end 142 77.59) (width 0.4) (layer "F.Cu") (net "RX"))
 (segment (start 141.96 77.63) (end 131 77.63) (width 0.4) (layer "F.Cu") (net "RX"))
 (segment (start 183.78 83.82) (end 162.56 83.82) (width 0.4) (layer "F.Cu") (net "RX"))
 (segment (start 142 77.59) (end 141.96 77.63) (width 0.4) (layer "F.Cu") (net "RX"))
 (segment (start 150.32 77.63) (end 141.96 77.63) (width 0.4) (layer "F.Cu") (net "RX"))
 (segment (start 162.56 83.82) (end 156.51 83.82) (width 0.4) (layer "F.Cu") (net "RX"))
 (segment (start 152.16 73.9) (end 152.16 75.96) (width 0.4) (layer "F.Cu") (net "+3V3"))
 (segment (start 152.16 75.96) (end 157.48 81.28) (width 0.4) (layer "F.Cu") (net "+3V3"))
 (segment (start 157.48 81.28) (end 162.56 81.28) (width 0.4) (layer "F.Cu") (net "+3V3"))
 (segment (start 160.2 93.9) (end 160.38 93.72) (width 0.4) (layer "B.Cu") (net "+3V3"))
 (segment (start 181.78 81.28) (end 162.56 81.28) (width 0.4) (layer "B.Cu") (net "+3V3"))
 (segment (start 184.66 84.16) (end 181.78 81.28) (width 0.4) (layer "B.Cu") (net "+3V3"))
 (segment (start 160.38 81.32) (end 160.42 81.28) (width 0.4) (layer "B.Cu") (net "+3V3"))
 (segment (start 158.58 93.9) (end 160.2 93.9) (width 0.4) (layer "B.Cu") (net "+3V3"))
 (segment (start 160.38 93.72) (end 160.38 81.32) (width 0.4) (layer "B.Cu") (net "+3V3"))
 (segment (start 184.66 93.24) (end 184.66 84.16) (width 0.4) (layer "B.Cu") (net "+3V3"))
 (segment (start 160.42 81.28) (end 162.56 81.28) (width 0.4) (layer "B.Cu") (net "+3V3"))
 (segment (start 162.28 81) (end 162.56 81.28) (width 0.4) (layer "B.Cu") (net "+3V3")))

